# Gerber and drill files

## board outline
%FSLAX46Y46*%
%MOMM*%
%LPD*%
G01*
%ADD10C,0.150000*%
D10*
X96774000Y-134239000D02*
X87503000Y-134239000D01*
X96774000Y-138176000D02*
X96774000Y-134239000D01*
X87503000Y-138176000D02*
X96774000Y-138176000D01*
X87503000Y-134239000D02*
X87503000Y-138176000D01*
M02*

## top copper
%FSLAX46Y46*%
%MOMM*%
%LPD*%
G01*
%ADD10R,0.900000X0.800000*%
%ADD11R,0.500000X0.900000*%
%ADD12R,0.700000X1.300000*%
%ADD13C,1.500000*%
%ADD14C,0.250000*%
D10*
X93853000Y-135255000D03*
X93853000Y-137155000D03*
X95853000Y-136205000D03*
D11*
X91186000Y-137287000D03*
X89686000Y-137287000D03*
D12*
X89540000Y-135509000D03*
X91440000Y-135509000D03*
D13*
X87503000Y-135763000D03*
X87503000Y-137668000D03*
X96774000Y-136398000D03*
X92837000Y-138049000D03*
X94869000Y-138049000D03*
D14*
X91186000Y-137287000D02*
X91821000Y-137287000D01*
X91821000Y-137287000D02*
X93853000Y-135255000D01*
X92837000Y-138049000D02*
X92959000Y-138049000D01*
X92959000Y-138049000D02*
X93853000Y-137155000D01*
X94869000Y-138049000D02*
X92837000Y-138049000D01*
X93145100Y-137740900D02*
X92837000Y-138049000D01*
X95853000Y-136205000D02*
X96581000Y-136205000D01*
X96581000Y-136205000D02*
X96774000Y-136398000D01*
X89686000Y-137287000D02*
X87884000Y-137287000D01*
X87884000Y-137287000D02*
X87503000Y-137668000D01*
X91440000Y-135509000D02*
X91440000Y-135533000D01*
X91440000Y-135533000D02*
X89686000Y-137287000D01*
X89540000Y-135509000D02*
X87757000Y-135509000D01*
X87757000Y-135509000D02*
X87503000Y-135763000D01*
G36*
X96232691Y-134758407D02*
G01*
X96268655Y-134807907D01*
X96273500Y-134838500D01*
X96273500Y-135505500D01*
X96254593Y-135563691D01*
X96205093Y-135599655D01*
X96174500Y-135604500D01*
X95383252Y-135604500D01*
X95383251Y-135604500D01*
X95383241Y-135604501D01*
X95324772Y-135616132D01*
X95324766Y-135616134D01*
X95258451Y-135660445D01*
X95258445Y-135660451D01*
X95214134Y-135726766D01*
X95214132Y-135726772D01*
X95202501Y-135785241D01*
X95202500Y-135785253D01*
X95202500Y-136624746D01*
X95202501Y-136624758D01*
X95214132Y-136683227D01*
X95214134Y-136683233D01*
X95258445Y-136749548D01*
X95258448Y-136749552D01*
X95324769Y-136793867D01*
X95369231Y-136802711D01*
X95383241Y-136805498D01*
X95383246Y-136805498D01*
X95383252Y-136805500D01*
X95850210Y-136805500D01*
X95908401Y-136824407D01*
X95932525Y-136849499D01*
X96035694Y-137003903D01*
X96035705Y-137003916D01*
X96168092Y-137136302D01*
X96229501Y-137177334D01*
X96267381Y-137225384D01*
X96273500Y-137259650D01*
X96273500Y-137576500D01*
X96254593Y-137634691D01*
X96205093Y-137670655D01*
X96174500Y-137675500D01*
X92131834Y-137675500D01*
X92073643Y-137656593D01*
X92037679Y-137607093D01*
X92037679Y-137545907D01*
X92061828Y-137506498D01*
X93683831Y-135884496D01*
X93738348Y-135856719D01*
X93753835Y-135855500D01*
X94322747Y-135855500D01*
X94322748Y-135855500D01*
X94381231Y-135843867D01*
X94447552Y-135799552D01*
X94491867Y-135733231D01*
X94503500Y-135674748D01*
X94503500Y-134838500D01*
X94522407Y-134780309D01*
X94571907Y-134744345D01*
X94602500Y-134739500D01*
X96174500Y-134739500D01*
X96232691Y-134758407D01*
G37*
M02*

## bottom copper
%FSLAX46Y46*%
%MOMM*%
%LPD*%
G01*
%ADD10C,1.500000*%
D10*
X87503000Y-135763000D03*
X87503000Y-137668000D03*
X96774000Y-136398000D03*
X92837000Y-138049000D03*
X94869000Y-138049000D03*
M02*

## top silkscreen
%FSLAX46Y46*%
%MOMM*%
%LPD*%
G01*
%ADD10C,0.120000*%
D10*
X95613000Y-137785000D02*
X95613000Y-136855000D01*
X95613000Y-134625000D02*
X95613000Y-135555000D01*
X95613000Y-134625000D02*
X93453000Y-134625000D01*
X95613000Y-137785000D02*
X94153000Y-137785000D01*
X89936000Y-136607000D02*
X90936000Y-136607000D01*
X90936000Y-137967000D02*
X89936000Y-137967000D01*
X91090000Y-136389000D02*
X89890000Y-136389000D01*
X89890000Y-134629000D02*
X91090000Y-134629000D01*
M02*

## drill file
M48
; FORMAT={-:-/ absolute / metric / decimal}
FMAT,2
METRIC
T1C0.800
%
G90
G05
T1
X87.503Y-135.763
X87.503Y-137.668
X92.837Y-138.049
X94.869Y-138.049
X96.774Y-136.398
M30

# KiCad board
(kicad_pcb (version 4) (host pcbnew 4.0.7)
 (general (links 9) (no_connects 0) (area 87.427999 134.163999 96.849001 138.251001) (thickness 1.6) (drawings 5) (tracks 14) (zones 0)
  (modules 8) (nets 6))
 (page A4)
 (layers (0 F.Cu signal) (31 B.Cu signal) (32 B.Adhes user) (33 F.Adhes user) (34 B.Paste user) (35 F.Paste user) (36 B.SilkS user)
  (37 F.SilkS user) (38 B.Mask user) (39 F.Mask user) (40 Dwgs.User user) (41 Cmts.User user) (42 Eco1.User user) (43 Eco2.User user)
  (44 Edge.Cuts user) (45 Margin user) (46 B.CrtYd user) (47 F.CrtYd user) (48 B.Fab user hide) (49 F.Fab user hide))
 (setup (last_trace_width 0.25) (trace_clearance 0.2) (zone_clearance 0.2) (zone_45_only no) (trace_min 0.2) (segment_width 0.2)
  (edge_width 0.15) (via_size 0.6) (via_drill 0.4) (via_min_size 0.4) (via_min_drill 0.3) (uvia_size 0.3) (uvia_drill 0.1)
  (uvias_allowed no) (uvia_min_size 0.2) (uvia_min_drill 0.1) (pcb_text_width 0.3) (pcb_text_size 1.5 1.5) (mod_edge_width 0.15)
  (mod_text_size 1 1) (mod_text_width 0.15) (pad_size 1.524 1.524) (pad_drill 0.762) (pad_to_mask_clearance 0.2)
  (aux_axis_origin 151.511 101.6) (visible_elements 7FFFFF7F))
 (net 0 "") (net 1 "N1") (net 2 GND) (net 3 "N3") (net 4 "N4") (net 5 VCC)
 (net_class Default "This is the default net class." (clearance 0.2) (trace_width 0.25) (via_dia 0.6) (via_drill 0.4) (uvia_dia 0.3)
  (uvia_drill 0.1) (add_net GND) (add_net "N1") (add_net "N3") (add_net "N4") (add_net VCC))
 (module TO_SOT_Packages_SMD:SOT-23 (layer F.Cu) (at 94.853 136.205)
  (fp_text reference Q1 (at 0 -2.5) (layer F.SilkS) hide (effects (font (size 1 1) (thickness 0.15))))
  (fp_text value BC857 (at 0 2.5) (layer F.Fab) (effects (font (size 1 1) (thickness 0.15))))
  (fp_line (start 0.76 1.58) (end 0.76 0.65) (layer F.SilkS) (width 0.12))
  (fp_line (start 0.76 -1.58) (end 0.76 -0.65) (layer F.SilkS) (width 0.12))
  (fp_line (start 0.76 -1.58) (end -1.4 -1.58) (layer F.SilkS) (width 0.12))
  (fp_line (start 0.76 1.58) (end -0.7 1.58) (layer F.SilkS) (width 0.12))
  (pad 1 smd rect (at -1 -0.95) (size 0.9 0.8) (layers F.Cu F.Paste F.Mask) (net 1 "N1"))
  (pad 2 smd rect (at -1 0.95) (size 0.9 0.8) (layers F.Cu F.Paste F.Mask) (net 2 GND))
  (pad 3 smd rect (at 1 0) (size 0.9 0.8) (layers F.Cu F.Paste F.Mask) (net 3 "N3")))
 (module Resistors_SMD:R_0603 (layer F.Cu) (at 90.436 137.287 180)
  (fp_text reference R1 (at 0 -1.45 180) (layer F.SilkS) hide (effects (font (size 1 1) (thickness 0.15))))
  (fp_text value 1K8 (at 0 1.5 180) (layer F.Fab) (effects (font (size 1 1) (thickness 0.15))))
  (fp_line (start 0.5 0.68) (end -0.5 0.68) (layer F.SilkS) (width 0.12))
  (fp_line (start -0.5 -0.68) (end 0.5 -0.68) (layer F.SilkS) (width 0.12))
  (pad 1 smd rect (at -0.75 0 180) (size 0.5 0.9) (layers F.Cu F.Paste F.Mask) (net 1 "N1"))
  (pad 2 smd rect (at 0.75 0 180) (size 0.5 0.9) (layers F.Cu F.Paste F.Mask) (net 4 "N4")))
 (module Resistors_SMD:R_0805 (layer F.Cu) (at 90.49 135.509)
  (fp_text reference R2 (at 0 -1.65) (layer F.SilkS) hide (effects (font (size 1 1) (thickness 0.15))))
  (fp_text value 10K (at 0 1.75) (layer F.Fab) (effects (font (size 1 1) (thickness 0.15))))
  (fp_line (start 0.6 0.88) (end -0.6 0.88) (layer F.SilkS) (width 0.12))
  (fp_line (start -0.6 -0.88) (end 0.6 -0.88) (layer F.SilkS) (width 0.12))
  (pad 1 smd rect (at -0.95 0) (size 0.7 1.3) (layers F.Cu F.Paste F.Mask) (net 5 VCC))
  (pad 2 smd rect (at 0.95 0) (size 0.7 1.3) (layers F.Cu F.Paste F.Mask) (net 4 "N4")))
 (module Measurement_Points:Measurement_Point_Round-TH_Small (layer F.Cu) (at 87.503 135.763)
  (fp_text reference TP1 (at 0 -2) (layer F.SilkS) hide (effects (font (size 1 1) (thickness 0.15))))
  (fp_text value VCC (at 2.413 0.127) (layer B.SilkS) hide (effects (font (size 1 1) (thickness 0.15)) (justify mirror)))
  (pad 1 thru_hole circle (at 0 0) (size 1.5 1.5) (drill 0.8) (layers *.Cu *.Mask) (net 5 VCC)))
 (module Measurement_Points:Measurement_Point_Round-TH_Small (layer F.Cu) (at 87.503 137.668)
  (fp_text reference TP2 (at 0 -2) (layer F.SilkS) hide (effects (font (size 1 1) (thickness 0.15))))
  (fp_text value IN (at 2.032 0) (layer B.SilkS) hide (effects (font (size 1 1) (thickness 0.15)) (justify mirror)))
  (pad 1 thru_hole circle (at 0 0) (size 1.5 1.5) (drill 0.8) (layers *.Cu *.Mask) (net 4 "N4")))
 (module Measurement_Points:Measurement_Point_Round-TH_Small (layer F.Cu) (at 96.774 136.398)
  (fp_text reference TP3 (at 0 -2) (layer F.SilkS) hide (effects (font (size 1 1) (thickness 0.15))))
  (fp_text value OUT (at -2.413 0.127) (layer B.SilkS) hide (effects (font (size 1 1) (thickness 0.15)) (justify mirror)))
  (pad 1 thru_hole circle (at 0 0) (size 1.5 1.5) (drill 0.8) (layers *.Cu *.Mask) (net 3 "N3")))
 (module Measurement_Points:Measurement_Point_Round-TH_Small (layer F.Cu) (at 92.837 138.049)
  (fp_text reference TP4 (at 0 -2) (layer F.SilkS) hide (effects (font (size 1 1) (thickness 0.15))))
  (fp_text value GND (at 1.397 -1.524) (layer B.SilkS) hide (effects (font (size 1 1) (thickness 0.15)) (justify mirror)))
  (pad 1 thru_hole circle (at 0 0) (size 1.5 1.5) (drill 0.8) (layers *.Cu *.Mask) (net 2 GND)))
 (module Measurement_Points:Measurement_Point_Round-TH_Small (layer F.Cu) (at 94.869 138.049)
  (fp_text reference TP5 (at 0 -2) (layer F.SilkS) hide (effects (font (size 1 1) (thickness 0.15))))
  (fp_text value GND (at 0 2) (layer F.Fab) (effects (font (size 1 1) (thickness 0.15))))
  (pad 1 thru_hole circle (at 0 0) (size 1.5 1.5) (drill 0.8) (layers *.Cu *.Mask) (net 2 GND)))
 (gr_line (start 96.774 134.239) (end 87.503 134.239) (layer Edge.Cuts) (width 0.15))
 (gr_line (start 96.774 138.176) (end 96.774 134.239) (layer Edge.Cuts) (width 0.15))
 (gr_line (start 87.503 138.176) (end 96.774 138.176) (layer Edge.Cuts) (width 0.15))
 (gr_line (start 87.503 134.239) (end 87.503 138.176) (layer Edge.Cuts) (width 0.15))
 (segment (start 91.186 137.287) (end 91.821 137.287) (width 0.25) (layer F.Cu) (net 1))
 (segment (start 91.821 137.287) (end 93.853 135.255) (width 0.25) (layer F.Cu) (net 1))
 (segment (start 92.837 138.049) (end 92.959 138.049) (width 0.25) (layer F.Cu) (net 2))
 (segment (start 92.959 138.049) (end 93.853 137.155) (width 0.25) (layer F.Cu) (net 2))
 (segment (start 94.869 138.049) (end 92.837 138.049) (width 0.25) (layer F.Cu) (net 2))
 (segment (start 93.1451 137.7409) (end 92.837 138.049) (width 0.25) (layer F.Cu) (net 2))
 (segment (start 95.853 136.205) (end 96.581 136.205) (width 0.25) (layer F.Cu) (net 3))
 (segment (start 96.581 136.205) (end 96.774 136.398) (width 0.25) (layer F.Cu) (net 3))
 (segment (start 89.686 137.287) (end 87.884 137.287) (width 0.25) (layer F.Cu) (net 4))
 (segment (start 87.884 137.287) (end 87.503 137.668) (width 0.25) (layer F.Cu) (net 4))
 (segment (start 91.44 135.509) (end 91.44 135.533) (width 0.25) (layer F.Cu) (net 4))
 (segment (start 91.44 135.533) (end 89.686 137.287) (width 0.25) (layer F.Cu) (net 4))
 (segment (start 89.54 135.509) (end 87.757 135.509) (width 0.25) (layer F.Cu) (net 5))
 (segment (start 87.757 135.509) (end 87.503 135.763) (width 0.25) (layer F.Cu) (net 5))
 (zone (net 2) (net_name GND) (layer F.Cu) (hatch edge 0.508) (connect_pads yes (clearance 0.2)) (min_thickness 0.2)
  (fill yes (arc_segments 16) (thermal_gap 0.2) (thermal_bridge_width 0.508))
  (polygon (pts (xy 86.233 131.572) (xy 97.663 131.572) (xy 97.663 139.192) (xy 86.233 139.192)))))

